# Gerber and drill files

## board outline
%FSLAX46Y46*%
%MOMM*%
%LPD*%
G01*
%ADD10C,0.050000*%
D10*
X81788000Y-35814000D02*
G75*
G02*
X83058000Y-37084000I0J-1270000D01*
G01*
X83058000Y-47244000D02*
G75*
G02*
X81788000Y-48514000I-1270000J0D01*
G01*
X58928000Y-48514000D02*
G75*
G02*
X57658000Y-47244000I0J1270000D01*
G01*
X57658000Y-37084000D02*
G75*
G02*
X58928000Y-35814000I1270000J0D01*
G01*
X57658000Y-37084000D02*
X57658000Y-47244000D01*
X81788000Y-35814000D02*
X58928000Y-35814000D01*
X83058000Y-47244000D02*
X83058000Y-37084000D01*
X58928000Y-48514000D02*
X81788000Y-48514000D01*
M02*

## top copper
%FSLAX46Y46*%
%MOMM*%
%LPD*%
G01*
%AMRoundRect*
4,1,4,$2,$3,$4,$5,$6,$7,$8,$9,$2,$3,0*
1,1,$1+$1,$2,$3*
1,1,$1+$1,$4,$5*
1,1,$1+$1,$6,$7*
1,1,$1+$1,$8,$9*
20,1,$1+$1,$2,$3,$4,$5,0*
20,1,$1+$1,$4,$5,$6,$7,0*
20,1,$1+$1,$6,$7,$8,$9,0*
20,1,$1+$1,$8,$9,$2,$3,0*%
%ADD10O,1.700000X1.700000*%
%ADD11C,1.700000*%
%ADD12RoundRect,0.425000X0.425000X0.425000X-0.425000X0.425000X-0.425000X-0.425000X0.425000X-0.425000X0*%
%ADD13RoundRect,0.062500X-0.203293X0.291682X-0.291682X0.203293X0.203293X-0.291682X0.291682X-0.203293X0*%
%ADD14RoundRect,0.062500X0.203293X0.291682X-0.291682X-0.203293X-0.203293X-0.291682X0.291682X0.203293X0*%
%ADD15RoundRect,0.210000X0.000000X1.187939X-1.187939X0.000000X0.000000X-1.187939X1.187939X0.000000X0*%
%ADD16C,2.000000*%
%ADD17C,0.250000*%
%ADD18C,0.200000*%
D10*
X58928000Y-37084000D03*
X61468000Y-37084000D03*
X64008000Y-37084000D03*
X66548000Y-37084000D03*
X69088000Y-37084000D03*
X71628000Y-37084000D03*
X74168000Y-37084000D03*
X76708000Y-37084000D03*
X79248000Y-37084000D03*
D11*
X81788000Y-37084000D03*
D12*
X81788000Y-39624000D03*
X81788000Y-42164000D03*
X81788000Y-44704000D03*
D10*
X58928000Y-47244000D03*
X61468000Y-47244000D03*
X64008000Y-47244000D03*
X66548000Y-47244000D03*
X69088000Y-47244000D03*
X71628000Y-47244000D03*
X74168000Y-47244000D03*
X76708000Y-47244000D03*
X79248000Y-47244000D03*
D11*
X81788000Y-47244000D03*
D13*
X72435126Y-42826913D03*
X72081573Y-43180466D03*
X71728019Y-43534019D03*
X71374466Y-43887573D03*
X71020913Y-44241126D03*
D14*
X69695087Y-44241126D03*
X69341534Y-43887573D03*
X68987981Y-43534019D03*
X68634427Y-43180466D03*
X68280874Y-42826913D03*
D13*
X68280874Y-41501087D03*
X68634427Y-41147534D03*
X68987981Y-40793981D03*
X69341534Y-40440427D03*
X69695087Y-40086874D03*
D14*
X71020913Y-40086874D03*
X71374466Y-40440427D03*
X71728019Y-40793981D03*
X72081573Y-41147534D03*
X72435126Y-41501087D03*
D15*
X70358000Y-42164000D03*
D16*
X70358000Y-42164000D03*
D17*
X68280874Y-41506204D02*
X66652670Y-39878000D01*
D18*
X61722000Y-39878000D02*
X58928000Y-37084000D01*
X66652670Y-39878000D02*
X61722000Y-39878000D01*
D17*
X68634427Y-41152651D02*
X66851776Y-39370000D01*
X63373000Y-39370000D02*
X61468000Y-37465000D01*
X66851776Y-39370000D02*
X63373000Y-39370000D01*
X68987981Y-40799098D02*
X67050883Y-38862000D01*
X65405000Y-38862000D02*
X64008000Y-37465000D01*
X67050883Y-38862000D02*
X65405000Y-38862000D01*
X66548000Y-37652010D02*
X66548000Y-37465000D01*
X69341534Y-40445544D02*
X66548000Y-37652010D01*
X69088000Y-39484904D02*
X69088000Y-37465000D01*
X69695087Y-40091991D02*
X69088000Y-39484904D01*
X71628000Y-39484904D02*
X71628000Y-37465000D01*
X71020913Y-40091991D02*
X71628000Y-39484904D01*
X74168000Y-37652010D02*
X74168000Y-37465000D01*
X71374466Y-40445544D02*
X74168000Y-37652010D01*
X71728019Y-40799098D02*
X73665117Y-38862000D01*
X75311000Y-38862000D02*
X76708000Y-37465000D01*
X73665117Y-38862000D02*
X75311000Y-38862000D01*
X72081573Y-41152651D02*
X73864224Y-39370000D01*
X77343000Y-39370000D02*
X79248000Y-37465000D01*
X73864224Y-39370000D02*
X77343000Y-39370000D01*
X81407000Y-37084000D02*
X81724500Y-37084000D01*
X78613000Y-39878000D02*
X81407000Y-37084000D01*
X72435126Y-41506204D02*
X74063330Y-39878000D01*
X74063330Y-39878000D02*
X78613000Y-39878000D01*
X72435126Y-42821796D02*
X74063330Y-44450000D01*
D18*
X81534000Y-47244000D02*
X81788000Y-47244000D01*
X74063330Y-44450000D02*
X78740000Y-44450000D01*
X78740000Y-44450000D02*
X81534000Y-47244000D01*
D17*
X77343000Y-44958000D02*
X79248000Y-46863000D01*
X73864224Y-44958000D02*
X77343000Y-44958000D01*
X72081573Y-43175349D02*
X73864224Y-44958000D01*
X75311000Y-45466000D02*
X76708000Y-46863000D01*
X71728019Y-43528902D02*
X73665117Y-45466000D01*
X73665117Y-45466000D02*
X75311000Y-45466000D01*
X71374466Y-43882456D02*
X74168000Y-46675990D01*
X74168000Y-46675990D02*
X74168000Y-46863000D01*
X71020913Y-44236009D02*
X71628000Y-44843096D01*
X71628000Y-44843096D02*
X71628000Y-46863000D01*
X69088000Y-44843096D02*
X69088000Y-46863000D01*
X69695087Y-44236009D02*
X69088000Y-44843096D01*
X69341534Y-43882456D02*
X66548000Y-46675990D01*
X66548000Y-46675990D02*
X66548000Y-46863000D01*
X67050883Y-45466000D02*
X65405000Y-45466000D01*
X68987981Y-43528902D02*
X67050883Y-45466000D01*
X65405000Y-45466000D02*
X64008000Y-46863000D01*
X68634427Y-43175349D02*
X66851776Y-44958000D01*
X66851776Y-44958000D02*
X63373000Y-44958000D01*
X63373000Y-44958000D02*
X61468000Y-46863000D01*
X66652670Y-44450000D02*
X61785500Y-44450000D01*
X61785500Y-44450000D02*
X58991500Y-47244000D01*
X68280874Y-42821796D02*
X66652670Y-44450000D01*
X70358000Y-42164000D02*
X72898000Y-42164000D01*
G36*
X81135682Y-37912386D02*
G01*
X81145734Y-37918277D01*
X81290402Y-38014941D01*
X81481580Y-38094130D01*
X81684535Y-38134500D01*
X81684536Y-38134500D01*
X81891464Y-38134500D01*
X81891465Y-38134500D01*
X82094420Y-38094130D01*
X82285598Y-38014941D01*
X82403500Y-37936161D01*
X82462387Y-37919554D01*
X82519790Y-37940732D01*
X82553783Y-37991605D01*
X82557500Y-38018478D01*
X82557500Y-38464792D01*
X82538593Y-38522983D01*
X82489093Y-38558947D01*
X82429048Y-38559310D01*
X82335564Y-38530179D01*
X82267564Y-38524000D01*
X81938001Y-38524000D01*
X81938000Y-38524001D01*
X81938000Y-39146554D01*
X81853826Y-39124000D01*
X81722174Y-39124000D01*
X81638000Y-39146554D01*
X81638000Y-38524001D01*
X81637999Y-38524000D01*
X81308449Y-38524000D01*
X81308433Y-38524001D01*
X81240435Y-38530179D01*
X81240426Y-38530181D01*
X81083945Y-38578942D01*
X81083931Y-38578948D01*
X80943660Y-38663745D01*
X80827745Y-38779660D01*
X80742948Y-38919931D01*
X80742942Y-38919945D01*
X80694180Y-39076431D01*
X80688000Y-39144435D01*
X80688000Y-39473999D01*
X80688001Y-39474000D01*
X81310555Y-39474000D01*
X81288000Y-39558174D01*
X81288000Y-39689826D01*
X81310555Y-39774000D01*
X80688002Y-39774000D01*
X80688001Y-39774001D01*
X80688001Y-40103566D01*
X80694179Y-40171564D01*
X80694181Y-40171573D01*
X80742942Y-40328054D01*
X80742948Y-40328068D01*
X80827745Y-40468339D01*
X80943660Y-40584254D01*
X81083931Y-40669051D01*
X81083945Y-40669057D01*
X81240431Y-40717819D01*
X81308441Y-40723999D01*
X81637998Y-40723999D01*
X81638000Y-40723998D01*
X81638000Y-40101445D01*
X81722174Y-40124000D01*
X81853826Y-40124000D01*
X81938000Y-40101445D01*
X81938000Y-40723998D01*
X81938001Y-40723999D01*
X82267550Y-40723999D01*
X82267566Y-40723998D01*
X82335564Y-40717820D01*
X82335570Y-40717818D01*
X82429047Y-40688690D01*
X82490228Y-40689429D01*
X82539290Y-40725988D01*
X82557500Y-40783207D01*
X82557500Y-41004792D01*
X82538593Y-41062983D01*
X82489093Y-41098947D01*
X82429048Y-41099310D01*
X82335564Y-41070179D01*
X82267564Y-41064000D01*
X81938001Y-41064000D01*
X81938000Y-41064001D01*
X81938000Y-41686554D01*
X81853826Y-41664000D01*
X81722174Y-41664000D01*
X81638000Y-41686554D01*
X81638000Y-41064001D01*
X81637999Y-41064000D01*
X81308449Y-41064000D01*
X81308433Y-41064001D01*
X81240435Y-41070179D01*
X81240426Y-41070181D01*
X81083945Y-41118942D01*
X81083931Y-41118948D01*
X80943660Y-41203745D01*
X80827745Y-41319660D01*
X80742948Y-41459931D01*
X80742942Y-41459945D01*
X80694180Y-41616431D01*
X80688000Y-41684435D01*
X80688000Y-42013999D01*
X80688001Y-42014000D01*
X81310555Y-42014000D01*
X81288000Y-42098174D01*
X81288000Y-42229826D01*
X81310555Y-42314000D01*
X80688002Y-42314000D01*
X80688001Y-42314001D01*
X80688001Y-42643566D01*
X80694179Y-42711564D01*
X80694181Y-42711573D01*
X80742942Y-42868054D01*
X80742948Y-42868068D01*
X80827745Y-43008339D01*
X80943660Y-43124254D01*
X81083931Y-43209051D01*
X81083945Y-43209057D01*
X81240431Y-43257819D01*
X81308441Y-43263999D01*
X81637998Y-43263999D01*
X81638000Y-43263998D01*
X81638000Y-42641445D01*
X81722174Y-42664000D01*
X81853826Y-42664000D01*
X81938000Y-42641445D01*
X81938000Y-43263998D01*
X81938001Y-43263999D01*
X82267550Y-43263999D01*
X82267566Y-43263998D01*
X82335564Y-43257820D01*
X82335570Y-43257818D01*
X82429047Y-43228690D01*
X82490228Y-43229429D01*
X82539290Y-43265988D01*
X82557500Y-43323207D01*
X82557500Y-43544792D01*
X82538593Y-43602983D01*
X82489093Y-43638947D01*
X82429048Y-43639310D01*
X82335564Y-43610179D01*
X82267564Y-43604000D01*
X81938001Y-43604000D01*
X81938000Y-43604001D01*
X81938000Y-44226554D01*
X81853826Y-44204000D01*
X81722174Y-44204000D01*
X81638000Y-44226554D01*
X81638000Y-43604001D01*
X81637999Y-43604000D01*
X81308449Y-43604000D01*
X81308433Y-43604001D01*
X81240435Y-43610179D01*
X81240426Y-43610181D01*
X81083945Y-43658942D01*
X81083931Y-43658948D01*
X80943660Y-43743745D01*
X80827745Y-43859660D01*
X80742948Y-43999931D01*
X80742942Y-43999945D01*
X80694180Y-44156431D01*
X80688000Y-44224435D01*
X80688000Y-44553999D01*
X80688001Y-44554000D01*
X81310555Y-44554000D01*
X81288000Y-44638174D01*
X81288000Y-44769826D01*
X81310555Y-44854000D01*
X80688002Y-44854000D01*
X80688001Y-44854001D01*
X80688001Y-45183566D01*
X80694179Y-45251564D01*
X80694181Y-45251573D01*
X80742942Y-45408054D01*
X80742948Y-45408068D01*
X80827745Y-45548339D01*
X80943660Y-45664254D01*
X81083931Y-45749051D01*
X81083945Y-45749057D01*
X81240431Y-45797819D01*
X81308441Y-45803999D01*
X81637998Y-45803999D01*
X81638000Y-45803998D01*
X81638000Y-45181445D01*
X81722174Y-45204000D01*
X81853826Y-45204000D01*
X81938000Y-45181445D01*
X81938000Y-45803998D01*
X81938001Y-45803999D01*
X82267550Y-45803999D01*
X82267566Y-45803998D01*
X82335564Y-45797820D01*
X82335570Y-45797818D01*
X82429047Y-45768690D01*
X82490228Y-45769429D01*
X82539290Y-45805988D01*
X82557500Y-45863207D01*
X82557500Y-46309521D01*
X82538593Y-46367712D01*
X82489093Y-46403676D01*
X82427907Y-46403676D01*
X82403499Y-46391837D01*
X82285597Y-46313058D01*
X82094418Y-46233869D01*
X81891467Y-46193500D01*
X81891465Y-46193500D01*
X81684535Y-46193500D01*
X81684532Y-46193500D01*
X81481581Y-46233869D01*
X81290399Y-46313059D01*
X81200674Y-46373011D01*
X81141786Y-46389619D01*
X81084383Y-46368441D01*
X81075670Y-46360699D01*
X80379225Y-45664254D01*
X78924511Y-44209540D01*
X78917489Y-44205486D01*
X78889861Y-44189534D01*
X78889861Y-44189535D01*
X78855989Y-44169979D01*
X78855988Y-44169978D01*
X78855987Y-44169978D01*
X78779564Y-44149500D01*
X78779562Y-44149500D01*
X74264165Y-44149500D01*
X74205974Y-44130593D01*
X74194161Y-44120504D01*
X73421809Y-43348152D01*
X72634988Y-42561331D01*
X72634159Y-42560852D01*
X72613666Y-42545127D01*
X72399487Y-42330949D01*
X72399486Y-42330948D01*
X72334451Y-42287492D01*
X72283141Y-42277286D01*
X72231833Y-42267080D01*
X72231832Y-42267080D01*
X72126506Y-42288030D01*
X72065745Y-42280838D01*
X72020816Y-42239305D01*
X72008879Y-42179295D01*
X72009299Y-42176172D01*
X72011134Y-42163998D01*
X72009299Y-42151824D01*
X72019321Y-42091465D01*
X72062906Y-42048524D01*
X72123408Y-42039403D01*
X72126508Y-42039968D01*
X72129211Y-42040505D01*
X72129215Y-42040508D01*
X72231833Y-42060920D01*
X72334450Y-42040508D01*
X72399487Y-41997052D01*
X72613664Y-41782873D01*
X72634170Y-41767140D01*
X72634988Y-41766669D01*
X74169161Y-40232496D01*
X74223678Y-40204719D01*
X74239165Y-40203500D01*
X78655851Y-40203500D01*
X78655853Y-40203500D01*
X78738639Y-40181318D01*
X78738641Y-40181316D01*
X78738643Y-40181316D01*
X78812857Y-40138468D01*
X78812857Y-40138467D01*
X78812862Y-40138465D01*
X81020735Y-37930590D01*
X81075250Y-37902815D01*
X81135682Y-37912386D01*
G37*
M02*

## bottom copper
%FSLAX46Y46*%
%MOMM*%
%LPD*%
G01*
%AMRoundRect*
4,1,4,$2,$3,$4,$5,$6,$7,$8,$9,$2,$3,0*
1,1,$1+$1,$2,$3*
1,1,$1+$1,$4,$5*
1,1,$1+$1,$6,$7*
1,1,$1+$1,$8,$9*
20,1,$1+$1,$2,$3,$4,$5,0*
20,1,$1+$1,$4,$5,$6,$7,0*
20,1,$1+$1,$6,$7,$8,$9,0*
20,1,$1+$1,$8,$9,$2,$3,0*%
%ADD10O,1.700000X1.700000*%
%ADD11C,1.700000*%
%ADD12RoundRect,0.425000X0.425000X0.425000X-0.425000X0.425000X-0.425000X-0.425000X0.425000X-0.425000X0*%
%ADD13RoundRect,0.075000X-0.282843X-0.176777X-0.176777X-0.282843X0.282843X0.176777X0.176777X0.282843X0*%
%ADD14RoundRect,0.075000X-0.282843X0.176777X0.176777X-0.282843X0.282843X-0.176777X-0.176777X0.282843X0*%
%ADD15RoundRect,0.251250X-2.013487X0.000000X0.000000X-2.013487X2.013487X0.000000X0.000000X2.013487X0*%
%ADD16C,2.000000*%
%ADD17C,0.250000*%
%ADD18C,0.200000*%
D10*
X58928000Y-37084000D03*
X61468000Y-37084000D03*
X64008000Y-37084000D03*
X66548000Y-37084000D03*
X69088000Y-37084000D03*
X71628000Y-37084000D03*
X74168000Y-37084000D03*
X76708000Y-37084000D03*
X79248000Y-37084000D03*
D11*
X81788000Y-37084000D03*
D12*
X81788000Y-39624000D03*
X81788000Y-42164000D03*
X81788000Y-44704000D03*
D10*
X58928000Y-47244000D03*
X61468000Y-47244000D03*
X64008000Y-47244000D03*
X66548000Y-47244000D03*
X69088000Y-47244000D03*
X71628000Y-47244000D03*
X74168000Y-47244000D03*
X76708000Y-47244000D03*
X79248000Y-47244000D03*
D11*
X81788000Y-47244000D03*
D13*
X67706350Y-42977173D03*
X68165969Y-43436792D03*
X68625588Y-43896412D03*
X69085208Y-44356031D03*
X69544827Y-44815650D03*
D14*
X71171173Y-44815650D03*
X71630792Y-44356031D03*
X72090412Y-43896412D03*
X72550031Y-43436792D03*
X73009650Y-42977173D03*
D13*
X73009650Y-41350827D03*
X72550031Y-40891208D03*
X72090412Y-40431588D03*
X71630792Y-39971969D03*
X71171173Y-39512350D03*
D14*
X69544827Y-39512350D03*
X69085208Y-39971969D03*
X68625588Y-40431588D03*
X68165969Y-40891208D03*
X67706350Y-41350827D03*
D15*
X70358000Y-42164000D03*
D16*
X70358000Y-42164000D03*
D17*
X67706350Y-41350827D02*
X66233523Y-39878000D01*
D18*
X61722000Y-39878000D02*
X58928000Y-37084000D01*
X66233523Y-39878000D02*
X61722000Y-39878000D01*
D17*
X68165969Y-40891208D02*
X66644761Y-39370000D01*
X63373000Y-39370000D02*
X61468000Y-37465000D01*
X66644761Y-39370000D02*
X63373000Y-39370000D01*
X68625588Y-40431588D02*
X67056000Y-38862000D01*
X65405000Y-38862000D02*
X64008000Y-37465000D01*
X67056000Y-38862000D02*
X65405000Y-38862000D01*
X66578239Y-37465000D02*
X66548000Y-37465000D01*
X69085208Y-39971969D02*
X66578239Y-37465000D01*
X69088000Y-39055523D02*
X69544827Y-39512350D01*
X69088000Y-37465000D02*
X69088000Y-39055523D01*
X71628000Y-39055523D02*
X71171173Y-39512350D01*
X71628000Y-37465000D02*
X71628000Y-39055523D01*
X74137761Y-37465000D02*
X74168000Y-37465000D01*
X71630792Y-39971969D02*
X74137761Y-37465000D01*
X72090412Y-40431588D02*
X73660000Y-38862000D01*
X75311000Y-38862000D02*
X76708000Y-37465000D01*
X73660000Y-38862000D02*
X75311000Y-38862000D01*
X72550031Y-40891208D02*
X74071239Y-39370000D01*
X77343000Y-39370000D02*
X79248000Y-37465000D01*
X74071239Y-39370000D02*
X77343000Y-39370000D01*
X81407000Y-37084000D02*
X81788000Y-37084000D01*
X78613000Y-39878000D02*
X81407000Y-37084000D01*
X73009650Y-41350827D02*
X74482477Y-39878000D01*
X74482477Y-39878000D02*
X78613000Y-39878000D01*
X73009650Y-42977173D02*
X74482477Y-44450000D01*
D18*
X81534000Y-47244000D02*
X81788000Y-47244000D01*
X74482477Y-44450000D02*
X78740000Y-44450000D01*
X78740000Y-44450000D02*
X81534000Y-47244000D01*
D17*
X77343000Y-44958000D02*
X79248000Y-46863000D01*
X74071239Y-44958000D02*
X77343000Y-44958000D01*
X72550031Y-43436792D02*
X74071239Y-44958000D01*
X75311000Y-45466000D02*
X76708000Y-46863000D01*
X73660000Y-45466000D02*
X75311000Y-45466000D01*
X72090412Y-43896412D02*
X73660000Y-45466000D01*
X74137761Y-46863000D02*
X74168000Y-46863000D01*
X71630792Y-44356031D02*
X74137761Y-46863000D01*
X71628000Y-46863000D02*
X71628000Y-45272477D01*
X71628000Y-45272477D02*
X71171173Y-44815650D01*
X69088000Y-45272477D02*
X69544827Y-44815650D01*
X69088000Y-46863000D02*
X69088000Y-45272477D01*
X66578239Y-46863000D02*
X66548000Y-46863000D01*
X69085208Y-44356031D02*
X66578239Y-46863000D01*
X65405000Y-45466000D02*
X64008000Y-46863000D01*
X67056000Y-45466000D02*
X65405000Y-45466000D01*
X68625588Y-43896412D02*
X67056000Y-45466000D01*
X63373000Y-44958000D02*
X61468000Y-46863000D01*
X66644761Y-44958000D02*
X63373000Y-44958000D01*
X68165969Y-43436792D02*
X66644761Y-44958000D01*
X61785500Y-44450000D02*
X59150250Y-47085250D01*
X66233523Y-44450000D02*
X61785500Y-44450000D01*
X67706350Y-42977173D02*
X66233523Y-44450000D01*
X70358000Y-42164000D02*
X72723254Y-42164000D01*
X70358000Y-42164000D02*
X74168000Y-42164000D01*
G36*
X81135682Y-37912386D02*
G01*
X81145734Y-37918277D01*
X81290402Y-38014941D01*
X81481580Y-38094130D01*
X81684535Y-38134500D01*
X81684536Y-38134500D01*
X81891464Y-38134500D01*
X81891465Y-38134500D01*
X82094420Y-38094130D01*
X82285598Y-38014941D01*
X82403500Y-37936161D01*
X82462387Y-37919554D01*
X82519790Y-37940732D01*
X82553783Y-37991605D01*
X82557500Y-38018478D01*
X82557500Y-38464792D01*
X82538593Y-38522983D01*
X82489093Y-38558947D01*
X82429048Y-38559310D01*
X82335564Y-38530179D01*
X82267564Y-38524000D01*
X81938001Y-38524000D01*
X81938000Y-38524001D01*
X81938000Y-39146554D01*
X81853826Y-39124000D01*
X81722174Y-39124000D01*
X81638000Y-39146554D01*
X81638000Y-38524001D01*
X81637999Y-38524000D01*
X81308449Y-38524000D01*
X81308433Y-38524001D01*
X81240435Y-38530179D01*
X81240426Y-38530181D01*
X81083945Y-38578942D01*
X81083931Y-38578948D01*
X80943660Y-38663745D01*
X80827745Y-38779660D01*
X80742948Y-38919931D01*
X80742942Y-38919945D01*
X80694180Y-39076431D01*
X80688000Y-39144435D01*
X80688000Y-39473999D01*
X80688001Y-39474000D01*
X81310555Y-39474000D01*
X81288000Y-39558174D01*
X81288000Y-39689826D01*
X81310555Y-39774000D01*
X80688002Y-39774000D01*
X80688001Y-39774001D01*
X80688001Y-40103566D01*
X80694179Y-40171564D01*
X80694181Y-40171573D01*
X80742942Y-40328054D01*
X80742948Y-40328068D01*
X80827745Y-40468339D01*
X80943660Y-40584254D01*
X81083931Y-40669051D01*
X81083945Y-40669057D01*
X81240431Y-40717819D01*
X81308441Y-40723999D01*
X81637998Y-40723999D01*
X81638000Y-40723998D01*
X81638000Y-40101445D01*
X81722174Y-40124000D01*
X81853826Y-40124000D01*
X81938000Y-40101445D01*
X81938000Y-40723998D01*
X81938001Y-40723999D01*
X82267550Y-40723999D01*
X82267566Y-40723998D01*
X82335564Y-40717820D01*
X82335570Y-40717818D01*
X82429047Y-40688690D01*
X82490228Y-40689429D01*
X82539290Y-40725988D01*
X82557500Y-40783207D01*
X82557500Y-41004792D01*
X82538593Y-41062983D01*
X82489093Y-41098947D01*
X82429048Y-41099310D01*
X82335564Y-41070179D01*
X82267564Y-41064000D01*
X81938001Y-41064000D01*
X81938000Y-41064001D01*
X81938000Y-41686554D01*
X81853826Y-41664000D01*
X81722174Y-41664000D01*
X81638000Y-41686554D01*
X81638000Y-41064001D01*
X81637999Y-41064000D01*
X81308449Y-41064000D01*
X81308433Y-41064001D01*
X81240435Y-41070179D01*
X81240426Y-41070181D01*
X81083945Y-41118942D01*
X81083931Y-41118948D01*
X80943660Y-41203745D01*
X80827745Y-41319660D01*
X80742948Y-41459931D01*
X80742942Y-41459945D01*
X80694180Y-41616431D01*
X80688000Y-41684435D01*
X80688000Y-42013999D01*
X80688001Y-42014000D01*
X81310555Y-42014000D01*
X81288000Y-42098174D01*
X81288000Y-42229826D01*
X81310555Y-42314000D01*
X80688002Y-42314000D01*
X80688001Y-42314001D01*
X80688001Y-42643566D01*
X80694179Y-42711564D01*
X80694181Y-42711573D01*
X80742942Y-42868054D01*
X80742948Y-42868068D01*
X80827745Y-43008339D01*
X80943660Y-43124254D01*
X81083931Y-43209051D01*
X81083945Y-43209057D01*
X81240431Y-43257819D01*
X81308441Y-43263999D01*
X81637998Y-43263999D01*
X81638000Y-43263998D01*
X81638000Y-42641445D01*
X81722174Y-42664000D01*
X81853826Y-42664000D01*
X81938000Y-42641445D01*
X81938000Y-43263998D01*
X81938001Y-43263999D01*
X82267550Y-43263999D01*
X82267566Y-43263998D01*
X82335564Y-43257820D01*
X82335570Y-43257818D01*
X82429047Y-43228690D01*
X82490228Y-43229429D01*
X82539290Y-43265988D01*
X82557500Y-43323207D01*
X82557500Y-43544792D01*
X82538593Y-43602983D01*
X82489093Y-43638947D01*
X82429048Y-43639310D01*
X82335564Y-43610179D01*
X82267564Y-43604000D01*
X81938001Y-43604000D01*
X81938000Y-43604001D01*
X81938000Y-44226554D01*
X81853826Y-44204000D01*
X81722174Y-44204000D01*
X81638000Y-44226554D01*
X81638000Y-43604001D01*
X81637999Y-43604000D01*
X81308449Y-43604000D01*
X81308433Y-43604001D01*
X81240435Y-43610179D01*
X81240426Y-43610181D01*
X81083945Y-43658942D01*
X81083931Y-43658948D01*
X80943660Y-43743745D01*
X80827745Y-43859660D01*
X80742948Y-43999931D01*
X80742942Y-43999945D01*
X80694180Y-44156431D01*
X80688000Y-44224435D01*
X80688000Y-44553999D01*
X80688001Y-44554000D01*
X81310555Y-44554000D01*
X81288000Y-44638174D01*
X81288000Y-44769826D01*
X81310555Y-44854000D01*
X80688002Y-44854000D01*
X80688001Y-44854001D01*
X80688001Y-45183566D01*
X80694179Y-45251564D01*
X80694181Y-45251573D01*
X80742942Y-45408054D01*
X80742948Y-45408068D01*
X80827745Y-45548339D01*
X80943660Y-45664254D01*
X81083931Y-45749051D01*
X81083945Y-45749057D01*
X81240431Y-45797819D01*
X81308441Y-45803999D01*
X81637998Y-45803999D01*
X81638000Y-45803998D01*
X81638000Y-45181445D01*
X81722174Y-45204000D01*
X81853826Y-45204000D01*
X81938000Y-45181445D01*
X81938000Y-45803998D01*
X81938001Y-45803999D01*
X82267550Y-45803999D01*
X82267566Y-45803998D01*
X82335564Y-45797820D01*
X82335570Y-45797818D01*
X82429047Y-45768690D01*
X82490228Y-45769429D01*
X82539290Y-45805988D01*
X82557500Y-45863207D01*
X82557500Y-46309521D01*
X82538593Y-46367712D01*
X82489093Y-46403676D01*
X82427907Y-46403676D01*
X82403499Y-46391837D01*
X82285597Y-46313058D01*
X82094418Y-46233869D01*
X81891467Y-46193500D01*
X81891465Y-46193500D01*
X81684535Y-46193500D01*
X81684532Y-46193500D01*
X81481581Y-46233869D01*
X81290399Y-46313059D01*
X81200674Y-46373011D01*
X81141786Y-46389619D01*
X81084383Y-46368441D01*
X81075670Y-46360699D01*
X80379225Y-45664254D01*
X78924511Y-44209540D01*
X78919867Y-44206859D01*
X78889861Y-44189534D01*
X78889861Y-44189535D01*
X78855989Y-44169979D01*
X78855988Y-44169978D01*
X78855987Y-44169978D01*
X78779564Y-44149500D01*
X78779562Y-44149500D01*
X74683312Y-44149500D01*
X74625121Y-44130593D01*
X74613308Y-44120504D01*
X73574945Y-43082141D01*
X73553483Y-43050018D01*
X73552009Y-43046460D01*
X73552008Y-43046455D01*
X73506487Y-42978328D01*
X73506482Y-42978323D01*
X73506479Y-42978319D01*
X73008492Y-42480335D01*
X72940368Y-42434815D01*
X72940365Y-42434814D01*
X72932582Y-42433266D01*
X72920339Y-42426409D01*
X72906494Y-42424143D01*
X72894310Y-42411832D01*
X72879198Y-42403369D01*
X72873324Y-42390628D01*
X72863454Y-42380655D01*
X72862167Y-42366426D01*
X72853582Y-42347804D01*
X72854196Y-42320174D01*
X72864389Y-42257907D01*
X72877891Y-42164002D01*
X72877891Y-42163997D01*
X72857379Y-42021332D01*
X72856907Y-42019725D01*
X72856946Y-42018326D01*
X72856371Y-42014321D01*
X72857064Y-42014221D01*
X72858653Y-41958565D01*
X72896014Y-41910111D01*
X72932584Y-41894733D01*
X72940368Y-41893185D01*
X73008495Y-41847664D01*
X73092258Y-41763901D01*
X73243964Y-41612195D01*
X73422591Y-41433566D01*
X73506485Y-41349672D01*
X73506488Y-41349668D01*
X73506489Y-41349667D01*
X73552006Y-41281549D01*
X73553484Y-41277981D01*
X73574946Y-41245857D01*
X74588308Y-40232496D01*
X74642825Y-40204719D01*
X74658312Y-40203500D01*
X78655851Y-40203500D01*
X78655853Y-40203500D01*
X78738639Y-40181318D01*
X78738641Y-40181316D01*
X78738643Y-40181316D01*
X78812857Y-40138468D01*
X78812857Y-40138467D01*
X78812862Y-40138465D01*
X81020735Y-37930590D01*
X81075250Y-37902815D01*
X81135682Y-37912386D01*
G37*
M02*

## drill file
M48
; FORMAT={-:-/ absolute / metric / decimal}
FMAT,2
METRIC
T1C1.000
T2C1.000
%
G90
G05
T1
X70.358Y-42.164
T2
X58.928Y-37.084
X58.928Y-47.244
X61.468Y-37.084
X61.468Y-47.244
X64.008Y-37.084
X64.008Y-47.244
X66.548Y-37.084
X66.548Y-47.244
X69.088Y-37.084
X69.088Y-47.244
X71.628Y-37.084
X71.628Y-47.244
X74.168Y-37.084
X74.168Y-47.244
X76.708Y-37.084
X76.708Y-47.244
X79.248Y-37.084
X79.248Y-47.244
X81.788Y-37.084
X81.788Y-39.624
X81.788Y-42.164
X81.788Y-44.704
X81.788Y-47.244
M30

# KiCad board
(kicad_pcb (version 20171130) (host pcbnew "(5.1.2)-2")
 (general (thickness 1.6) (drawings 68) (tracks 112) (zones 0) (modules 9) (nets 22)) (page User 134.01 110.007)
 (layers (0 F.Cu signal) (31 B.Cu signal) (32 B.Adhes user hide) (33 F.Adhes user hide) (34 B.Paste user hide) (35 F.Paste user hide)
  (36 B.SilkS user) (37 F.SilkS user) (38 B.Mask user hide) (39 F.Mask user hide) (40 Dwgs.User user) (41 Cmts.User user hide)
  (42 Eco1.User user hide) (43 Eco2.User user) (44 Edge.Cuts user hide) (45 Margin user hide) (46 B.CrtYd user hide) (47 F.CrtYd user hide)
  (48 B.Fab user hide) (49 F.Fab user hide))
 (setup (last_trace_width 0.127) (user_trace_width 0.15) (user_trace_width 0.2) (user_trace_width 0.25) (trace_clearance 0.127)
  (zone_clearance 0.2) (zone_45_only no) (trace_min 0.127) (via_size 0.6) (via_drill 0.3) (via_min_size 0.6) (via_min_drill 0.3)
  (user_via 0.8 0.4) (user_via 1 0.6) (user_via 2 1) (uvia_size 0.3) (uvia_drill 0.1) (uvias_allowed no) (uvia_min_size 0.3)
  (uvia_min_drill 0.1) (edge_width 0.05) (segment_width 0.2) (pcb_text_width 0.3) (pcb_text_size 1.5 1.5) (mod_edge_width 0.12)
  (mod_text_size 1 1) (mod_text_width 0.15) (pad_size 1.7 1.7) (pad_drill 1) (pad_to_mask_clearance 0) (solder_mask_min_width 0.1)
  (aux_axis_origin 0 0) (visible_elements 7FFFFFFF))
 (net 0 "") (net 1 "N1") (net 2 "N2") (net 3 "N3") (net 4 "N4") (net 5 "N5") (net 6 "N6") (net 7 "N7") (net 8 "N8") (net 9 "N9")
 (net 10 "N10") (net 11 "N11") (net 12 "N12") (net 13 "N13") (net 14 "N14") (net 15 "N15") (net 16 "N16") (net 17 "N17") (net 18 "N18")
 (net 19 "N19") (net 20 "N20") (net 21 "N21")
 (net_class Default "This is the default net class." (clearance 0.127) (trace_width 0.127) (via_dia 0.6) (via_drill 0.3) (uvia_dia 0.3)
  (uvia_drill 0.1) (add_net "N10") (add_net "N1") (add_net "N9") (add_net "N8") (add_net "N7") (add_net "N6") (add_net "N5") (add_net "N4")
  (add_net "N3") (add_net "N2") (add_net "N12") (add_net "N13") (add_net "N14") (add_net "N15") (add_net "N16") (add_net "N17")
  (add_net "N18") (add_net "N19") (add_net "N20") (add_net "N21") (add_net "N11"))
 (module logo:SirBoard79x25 (layer B.Cu) (at 62.738 43.688)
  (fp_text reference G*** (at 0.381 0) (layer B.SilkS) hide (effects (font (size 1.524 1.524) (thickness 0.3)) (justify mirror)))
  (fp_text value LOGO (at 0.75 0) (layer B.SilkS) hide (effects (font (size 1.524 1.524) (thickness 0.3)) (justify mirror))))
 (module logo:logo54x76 (layer B.Cu) (at 76.708 42.164)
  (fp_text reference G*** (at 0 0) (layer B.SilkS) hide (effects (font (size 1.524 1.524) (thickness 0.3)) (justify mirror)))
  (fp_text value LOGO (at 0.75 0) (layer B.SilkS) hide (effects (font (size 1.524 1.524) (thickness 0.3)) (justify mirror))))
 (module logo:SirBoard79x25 (layer F.Cu) (at 62.738 43.688)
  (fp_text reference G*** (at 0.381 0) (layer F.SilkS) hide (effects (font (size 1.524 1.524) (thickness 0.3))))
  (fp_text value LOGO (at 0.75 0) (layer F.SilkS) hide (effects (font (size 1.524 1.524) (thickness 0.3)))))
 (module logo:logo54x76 (layer F.Cu) (at 76.708 42.164)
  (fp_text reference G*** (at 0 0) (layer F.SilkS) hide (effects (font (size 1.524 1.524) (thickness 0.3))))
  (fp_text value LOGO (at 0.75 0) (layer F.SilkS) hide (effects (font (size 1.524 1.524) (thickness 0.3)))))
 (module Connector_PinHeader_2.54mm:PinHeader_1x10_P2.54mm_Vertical (layer F.Cu) (at 81.788 37.084 270)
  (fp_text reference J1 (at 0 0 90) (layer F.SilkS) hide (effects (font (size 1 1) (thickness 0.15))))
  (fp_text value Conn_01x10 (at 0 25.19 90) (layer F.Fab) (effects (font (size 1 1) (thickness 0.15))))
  (pad 10 thru_hole oval (at 0 22.86 270) (size 1.7 1.7) (drill 1) (layers *.Cu *.Mask) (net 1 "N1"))
  (pad 9 thru_hole oval (at 0 20.32 270) (size 1.7 1.7) (drill 1) (layers *.Cu *.Mask) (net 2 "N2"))
  (pad 8 thru_hole oval (at 0 17.78 270) (size 1.7 1.7) (drill 1) (layers *.Cu *.Mask) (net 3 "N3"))
  (pad 7 thru_hole oval (at 0 15.24 270) (size 1.7 1.7) (drill 1) (layers *.Cu *.Mask) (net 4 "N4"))
  (pad 6 thru_hole oval (at 0 12.7 270) (size 1.7 1.7) (drill 1) (layers *.Cu *.Mask) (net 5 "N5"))
  (pad 5 thru_hole oval (at 0 10.16 270) (size 1.7 1.7) (drill 1) (layers *.Cu *.Mask) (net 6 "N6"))
  (pad 4 thru_hole oval (at 0 7.62 270) (size 1.7 1.7) (drill 1) (layers *.Cu *.Mask) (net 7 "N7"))
  (pad 3 thru_hole oval (at 0 5.08 270) (size 1.7 1.7) (drill 1) (layers *.Cu *.Mask) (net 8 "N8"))
  (pad 2 thru_hole oval (at 0 2.54 270) (size 1.7 1.7) (drill 1) (layers *.Cu *.Mask) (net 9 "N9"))
  (pad 1 thru_hole circle (at 0 0 270) (size 1.7 1.7) (drill 1) (layers *.Cu *.Mask) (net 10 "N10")))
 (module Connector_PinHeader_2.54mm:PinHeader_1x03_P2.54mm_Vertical (layer B.Cu) (at 81.788 39.624 180)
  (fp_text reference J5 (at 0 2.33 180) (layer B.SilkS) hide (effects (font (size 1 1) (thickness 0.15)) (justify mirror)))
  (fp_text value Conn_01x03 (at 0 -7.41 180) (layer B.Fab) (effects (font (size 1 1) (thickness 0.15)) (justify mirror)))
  (pad 1 thru_hole roundrect (at 0 0 180) (size 1.7 1.7) (drill 1) (layers *.Cu *.Mask) (roundrect_rratio 0.25) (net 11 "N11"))
  (pad 2 thru_hole roundrect (at 0 -2.54 180) (size 1.7 1.7) (drill 1) (layers *.Cu *.Mask) (roundrect_rratio 0.25) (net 11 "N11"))
  (pad 3 thru_hole roundrect (at 0 -5.08 180) (size 1.7 1.7) (drill 1) (layers *.Cu *.Mask) (roundrect_rratio 0.25) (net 11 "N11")))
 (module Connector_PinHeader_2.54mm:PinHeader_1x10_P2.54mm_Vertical (layer F.Cu) (at 81.788 47.244 270)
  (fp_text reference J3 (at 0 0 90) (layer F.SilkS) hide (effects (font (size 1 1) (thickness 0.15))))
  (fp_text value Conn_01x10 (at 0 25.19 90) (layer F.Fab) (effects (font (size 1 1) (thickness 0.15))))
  (pad 10 thru_hole oval (at 0 22.86 270) (size 1.7 1.7) (drill 1) (layers *.Cu *.Mask) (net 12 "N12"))
  (pad 9 thru_hole oval (at 0 20.32 270) (size 1.7 1.7) (drill 1) (layers *.Cu *.Mask) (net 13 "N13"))
  (pad 8 thru_hole oval (at 0 17.78 270) (size 1.7 1.7) (drill 1) (layers *.Cu *.Mask) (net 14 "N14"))
  (pad 7 thru_hole oval (at 0 15.24 270) (size 1.7 1.7) (drill 1) (layers *.Cu *.Mask) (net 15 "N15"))
  (pad 6 thru_hole oval (at 0 12.7 270) (size 1.7 1.7) (drill 1) (layers *.Cu *.Mask) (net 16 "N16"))
  (pad 5 thru_hole oval (at 0 10.16 270) (size 1.7 1.7) (drill 1) (layers *.Cu *.Mask) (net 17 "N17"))
  (pad 4 thru_hole oval (at 0 7.62 270) (size 1.7 1.7) (drill 1) (layers *.Cu *.Mask) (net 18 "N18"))
  (pad 3 thru_hole oval (at 0 5.08 270) (size 1.7 1.7) (drill 1) (layers *.Cu *.Mask) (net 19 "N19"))
  (pad 2 thru_hole oval (at 0 2.54 270) (size 1.7 1.7) (drill 1) (layers *.Cu *.Mask) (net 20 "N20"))
  (pad 1 thru_hole circle (at 0 0 270) (size 1.7 1.7) (drill 1) (layers *.Cu *.Mask) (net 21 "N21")))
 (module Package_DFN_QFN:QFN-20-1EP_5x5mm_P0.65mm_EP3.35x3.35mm (layer B.Cu) (at 70.358 42.164 315)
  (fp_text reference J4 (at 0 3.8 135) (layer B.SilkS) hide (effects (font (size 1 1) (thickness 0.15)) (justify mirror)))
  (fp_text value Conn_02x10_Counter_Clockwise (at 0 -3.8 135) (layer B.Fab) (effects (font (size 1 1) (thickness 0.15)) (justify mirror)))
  (pad 20 smd roundrect (at -1.3 2.45 315) (size 0.3 0.8) (layers B.Cu B.Paste B.Mask) (roundrect_rratio 0.25) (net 12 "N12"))
  (pad 19 smd roundrect (at -0.65 2.45 315) (size 0.3 0.8) (layers B.Cu B.Paste B.Mask) (roundrect_rratio 0.25) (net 13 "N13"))
  (pad 18 smd roundrect (at 0 2.45 315) (size 0.3 0.8) (layers B.Cu B.Paste B.Mask) (roundrect_rratio 0.25) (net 14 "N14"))
  (pad 17 smd roundrect (at 0.65 2.45 315) (size 0.3 0.8) (layers B.Cu B.Paste B.Mask) (roundrect_rratio 0.25) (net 15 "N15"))
  (pad 16 smd roundrect (at 1.3 2.45 315) (size 0.3 0.8) (layers B.Cu B.Paste B.Mask) (roundrect_rratio 0.25) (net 16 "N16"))
  (pad 15 smd roundrect (at 2.45 1.3 315) (size 0.8 0.3) (layers B.Cu B.Paste B.Mask) (roundrect_rratio 0.25) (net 17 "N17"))
  (pad 14 smd roundrect (at 2.45 0.65 315) (size 0.8 0.3) (layers B.Cu B.Paste B.Mask) (roundrect_rratio 0.25) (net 18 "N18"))
  (pad 13 smd roundrect (at 2.45 0 315) (size 0.8 0.3) (layers B.Cu B.Paste B.Mask) (roundrect_rratio 0.25) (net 19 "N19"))
  (pad 12 smd roundrect (at 2.45 -0.65 315) (size 0.8 0.3) (layers B.Cu B.Paste B.Mask) (roundrect_rratio 0.25) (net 20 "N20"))
  (pad 11 smd roundrect (at 2.45 -1.3 315) (size 0.8 0.3) (layers B.Cu B.Paste B.Mask) (roundrect_rratio 0.25) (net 21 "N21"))
  (pad 10 smd roundrect (at 1.3 -2.45 315) (size 0.3 0.8) (layers B.Cu B.Paste B.Mask) (roundrect_rratio 0.25) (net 10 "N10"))
  (pad 9 smd roundrect (at 0.65 -2.45 315) (size 0.3 0.8) (layers B.Cu B.Paste B.Mask) (roundrect_rratio 0.25) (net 9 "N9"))
  (pad 8 smd roundrect (at 0 -2.45 315) (size 0.3 0.8) (layers B.Cu B.Paste B.Mask) (roundrect_rratio 0.25) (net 8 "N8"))
  (pad 7 smd roundrect (at -0.65 -2.45 315) (size 0.3 0.8) (layers B.Cu B.Paste B.Mask) (roundrect_rratio 0.25) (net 7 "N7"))
  (pad 6 smd roundrect (at -1.3 -2.45 315) (size 0.3 0.8) (layers B.Cu B.Paste B.Mask) (roundrect_rratio 0.25) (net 6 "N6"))
  (pad 5 smd roundrect (at -2.45 -1.3 315) (size 0.8 0.3) (layers B.Cu B.Paste B.Mask) (roundrect_rratio 0.25) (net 5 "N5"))
  (pad 4 smd roundrect (at -2.45 -0.65 315) (size 0.8 0.3) (layers B.Cu B.Paste B.Mask) (roundrect_rratio 0.25) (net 4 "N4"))
  (pad 3 smd roundrect (at -2.45 0 315) (size 0.8 0.3) (layers B.Cu B.Paste B.Mask) (roundrect_rratio 0.25) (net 3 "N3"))
  (pad 2 smd roundrect (at -2.45 0.65 315) (size 0.8 0.3) (layers B.Cu B.Paste B.Mask) (roundrect_rratio 0.25) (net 2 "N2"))
  (pad 1 smd roundrect (at -2.45 1.3 315) (size 0.8 0.3) (layers B.Cu B.Paste B.Mask) (roundrect_rratio 0.25) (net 1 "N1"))
  (pad "" smd roundrect (at 0.84 -0.84 315) (size 1.35 1.35) (layers B.Paste) (roundrect_rratio 0.185185))
  (pad "" smd roundrect (at 0.84 0.84 315) (size 1.35 1.35) (layers B.Paste) (roundrect_rratio 0.185185))
  (pad "" smd roundrect (at -0.84 -0.84 315) (size 1.35 1.35) (layers B.Paste) (roundrect_rratio 0.185185))
  (pad "" smd roundrect (at -0.84 0.84 315) (size 1.35 1.35) (layers B.Paste) (roundrect_rratio 0.185185))
  (pad 21 smd roundrect (at 0 0 315) (size 3.35 3.35) (layers B.Cu B.Mask) (roundrect_rratio 0.075) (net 11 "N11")))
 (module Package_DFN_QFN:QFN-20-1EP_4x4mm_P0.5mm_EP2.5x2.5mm (layer F.Cu) (at 70.358 42.164 225)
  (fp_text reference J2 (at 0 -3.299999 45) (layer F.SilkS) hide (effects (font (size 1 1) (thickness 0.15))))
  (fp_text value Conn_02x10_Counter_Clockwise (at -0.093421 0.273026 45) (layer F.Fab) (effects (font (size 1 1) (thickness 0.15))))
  (pad 20 smd roundrect (at -1 -1.9375 225) (size 0.25 0.825) (layers F.Cu F.Paste F.Mask) (roundrect_rratio 0.25) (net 21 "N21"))
  (pad 19 smd roundrect (at -0.5 -1.9375 225) (size 0.25 0.825) (layers F.Cu F.Paste F.Mask) (roundrect_rratio 0.25) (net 20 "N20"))
  (pad 18 smd roundrect (at 0 -1.9375 225) (size 0.25 0.825) (layers F.Cu F.Paste F.Mask) (roundrect_rratio 0.25) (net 19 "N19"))
  (pad 17 smd roundrect (at 0.5 -1.9375 225) (size 0.25 0.825) (layers F.Cu F.Paste F.Mask) (roundrect_rratio 0.25) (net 18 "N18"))
  (pad 16 smd roundrect (at 1 -1.9375 225) (size 0.25 0.825) (layers F.Cu F.Paste F.Mask) (roundrect_rratio 0.25) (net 17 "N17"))
  (pad 15 smd roundrect (at 1.9375 -1 225) (size 0.825 0.25) (layers F.Cu F.Paste F.Mask) (roundrect_rratio 0.25) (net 16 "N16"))
  (pad 14 smd roundrect (at 1.9375 -0.5 225) (size 0.825 0.25) (layers F.Cu F.Paste F.Mask) (roundrect_rratio 0.25) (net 15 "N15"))
  (pad 13 smd roundrect (at 1.9375 0 225) (size 0.825 0.25) (layers F.Cu F.Paste F.Mask) (roundrect_rratio 0.25) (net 14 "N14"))
  (pad 12 smd roundrect (at 1.9375 0.5 225) (size 0.825 0.25) (layers F.Cu F.Paste F.Mask) (roundrect_rratio 0.25) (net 13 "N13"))
  (pad 11 smd roundrect (at 1.9375 1 225) (size 0.825 0.25) (layers F.Cu F.Paste F.Mask) (roundrect_rratio 0.25) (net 12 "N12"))
  (pad 10 smd roundrect (at 1 1.9375 225) (size 0.25 0.825) (layers F.Cu F.Paste F.Mask) (roundrect_rratio 0.25) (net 1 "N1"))
  (pad 9 smd roundrect (at 0.5 1.9375 225) (size 0.25 0.825) (layers F.Cu F.Paste F.Mask) (roundrect_rratio 0.25) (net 2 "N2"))
  (pad 8 smd roundrect (at 0 1.9375 225) (size 0.25 0.825) (layers F.Cu F.Paste F.Mask) (roundrect_rratio 0.25) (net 3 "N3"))
  (pad 7 smd roundrect (at -0.5 1.9375 225) (size 0.25 0.825) (layers F.Cu F.Paste F.Mask) (roundrect_rratio 0.25) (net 4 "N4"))
  (pad 6 smd roundrect (at -1 1.9375 225) (size 0.25 0.825) (layers F.Cu F.Paste F.Mask) (roundrect_rratio 0.25) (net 5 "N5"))
  (pad 5 smd roundrect (at -1.9375 1 225) (size 0.825 0.25) (layers F.Cu F.Paste F.Mask) (roundrect_rratio 0.25) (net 6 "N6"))
  (pad 4 smd roundrect (at -1.9375 0.5 225) (size 0.825 0.25) (layers F.Cu F.Paste F.Mask) (roundrect_rratio 0.25) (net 7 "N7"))
  (pad 3 smd roundrect (at -1.9375 0 225) (size 0.825 0.25) (layers F.Cu F.Paste F.Mask) (roundrect_rratio 0.25) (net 8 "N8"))
  (pad 2 smd roundrect (at -1.9375 -0.5 225) (size 0.825 0.25) (layers F.Cu F.Paste F.Mask) (roundrect_rratio 0.25) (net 9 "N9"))
  (pad 1 smd roundrect (at -1.9375 -1 225) (size 0.825 0.25) (layers F.Cu F.Paste F.Mask) (roundrect_rratio 0.25) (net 10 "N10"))
  (pad "" smd roundrect (at 0.625 0.625 225) (size 1.01 1.01) (layers F.Paste) (roundrect_rratio 0.247525))
  (pad "" smd roundrect (at 0.625 -0.625 225) (size 1.01 1.01) (layers F.Paste) (roundrect_rratio 0.247525))
  (pad "" smd roundrect (at -0.625 0.625 225) (size 1.01 1.01) (layers F.Paste) (roundrect_rratio 0.247525))
  (pad "" smd roundrect (at -0.625 -0.625 225) (size 1.01 1.01) (layers F.Paste) (roundrect_rratio 0.247525))
  (pad 21 smd roundrect (at 0 0 225) (size 2.1 2.1) (layers F.Cu F.Mask) (roundrect_rratio 0.1) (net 11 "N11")))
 (gr_arc (start 81.788 37.084) (end 83.058 37.084) (angle -90) (layer Edge.Cuts) (width 0.05))
 (gr_arc (start 81.788 47.244) (end 81.788 48.514) (angle -90) (layer Edge.Cuts) (width 0.05))
 (gr_arc (start 58.928 47.244) (end 57.658 47.244) (angle -90) (layer Edge.Cuts) (width 0.05))
 (gr_arc (start 58.928 37.084) (end 58.928 35.814) (angle -90) (layer Edge.Cuts) (width 0.05))
 (gr_line (start 57.658 37.084) (end 57.658 47.244) (layer Edge.Cuts) (width 0.05))
 (gr_line (start 81.788 35.814) (end 58.928 35.814) (layer Edge.Cuts) (width 0.05))
 (gr_line (start 83.058 47.244) (end 83.058 37.084) (layer Edge.Cuts) (width 0.05))
 (gr_line (start 58.928 48.514) (end 81.788 48.514) (layer Edge.Cuts) (width 0.05))
 (segment (start 68.280874 41.506204) (end 66.65267 39.878) (width 0.25) (layer F.Cu) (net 1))
 (segment (start 67.70635 41.350827) (end 66.233523 39.878) (width 0.25) (layer B.Cu) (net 1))
 (segment (start 61.722 39.878) (end 58.928 37.084) (width 0.2) (layer B.Cu) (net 1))
 (segment (start 61.722 39.878) (end 58.928 37.084) (width 0.2) (layer F.Cu) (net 1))
 (segment (start 66.65267 39.878) (end 61.722 39.878) (width 0.2) (layer F.Cu) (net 1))
 (segment (start 66.233523 39.878) (end 61.722 39.878) (width 0.2) (layer B.Cu) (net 1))
 (segment (start 68.634427 41.152651) (end 66.851776 39.37) (width 0.25) (layer F.Cu) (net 2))
 (segment (start 63.373 39.37) (end 61.468 37.465) (width 0.25) (layer F.Cu) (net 2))
 (segment (start 66.851776 39.37) (end 63.373 39.37) (width 0.25) (layer F.Cu) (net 2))
 (segment (start 68.165969 40.891208) (end 66.644761 39.37) (width 0.25) (layer B.Cu) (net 2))
 (segment (start 63.373 39.37) (end 61.468 37.465) (width 0.25) (layer B.Cu) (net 2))
 (segment (start 66.644761 39.37) (end 63.373 39.37) (width 0.25) (layer B.Cu) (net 2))
 (segment (start 68.987981 40.799098) (end 67.050883 38.862) (width 0.25) (layer F.Cu) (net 3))
 (segment (start 65.405 38.862) (end 64.008 37.465) (width 0.25) (layer F.Cu) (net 3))
 (segment (start 67.050883 38.862) (end 65.405 38.862) (width 0.25) (layer F.Cu) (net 3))
 (segment (start 68.625588 40.431588) (end 67.056 38.862) (width 0.25) (layer B.Cu) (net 3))
 (segment (start 65.405 38.862) (end 64.008 37.465) (width 0.25) (layer B.Cu) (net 3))
 (segment (start 67.056 38.862) (end 65.405 38.862) (width 0.25) (layer B.Cu) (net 3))
 (segment (start 66.548 37.65201) (end 66.548 37.465) (width 0.25) (layer F.Cu) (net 4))
 (segment (start 69.341534 40.445544) (end 66.548 37.65201) (width 0.25) (layer F.Cu) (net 4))
 (segment (start 66.578239 37.465) (end 66.548 37.465) (width 0.25) (layer B.Cu) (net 4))
 (segment (start 69.085208 39.971969) (end 66.578239 37.465) (width 0.25) (layer B.Cu) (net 4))
 (segment (start 69.088 39.484904) (end 69.088 37.465) (width 0.25) (layer F.Cu) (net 5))
 (segment (start 69.695087 40.091991) (end 69.088 39.484904) (width 0.25) (layer F.Cu) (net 5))
 (segment (start 69.088 39.055523) (end 69.544827 39.51235) (width 0.25) (layer B.Cu) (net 5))
 (segment (start 69.088 37.465) (end 69.088 39.055523) (width 0.25) (layer B.Cu) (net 5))
 (segment (start 71.628 39.484904) (end 71.628 37.465) (width 0.25) (layer F.Cu) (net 6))
 (segment (start 71.020913 40.091991) (end 71.628 39.484904) (width 0.25) (layer F.Cu) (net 6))
 (segment (start 71.628 39.055523) (end 71.171173 39.51235) (width 0.25) (layer B.Cu) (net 6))
 (segment (start 71.628 37.465) (end 71.628 39.055523) (width 0.25) (layer B.Cu) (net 6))
 (segment (start 74.168 37.65201) (end 74.168 37.465) (width 0.25) (layer F.Cu) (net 7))
 (segment (start 71.374466 40.445544) (end 74.168 37.65201) (width 0.25) (layer F.Cu) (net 7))
 (segment (start 74.137761 37.465) (end 74.168 37.465) (width 0.25) (layer B.Cu) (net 7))
 (segment (start 71.630792 39.971969) (end 74.137761 37.465) (width 0.25) (layer B.Cu) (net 7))
 (segment (start 71.728019 40.799098) (end 73.665117 38.862) (width 0.25) (layer F.Cu) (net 8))
 (segment (start 75.311 38.862) (end 76.708 37.465) (width 0.25) (layer F.Cu) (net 8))
 (segment (start 73.665117 38.862) (end 75.311 38.862) (width 0.25) (layer F.Cu) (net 8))
 (segment (start 72.090412 40.431588) (end 73.66 38.862) (width 0.25) (layer B.Cu) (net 8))
 (segment (start 75.311 38.862) (end 76.708 37.465) (width 0.25) (layer B.Cu) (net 8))
 (segment (start 73.66 38.862) (end 75.311 38.862) (width 0.25) (layer B.Cu) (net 8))
 (segment (start 72.081573 41.152651) (end 73.864224 39.37) (width 0.25) (layer F.Cu) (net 9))
 (segment (start 77.343 39.37) (end 79.248 37.465) (width 0.25) (layer F.Cu) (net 9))
 (segment (start 73.864224 39.37) (end 77.343 39.37) (width 0.25) (layer F.Cu) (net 9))
 (segment (start 72.550031 40.891208) (end 74.071239 39.37) (width 0.25) (layer B.Cu) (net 9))
 (segment (start 77.343 39.37) (end 79.248 37.465) (width 0.25) (layer B.Cu) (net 9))
 (segment (start 74.071239 39.37) (end 77.343 39.37) (width 0.25) (layer B.Cu) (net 9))
 (segment (start 81.407 37.084) (end 81.788 37.084) (width 0.25) (layer B.Cu) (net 10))
 (segment (start 78.613 39.878) (end 81.407 37.084) (width 0.25) (layer B.Cu) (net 10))
 (segment (start 73.00965 41.350827) (end 74.482477 39.878) (width 0.25) (layer B.Cu) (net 10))
 (segment (start 74.482477 39.878) (end 78.613 39.878) (width 0.25) (layer B.Cu) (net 10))
 (segment (start 81.407 37.084) (end 81.7245 37.084) (width 0.25) (layer F.Cu) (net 10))
 (segment (start 78.613 39.878) (end 81.407 37.084) (width 0.25) (layer F.Cu) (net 10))
 (segment (start 72.435126 41.506204) (end 74.06333 39.878) (width 0.25) (layer F.Cu) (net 10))
 (segment (start 74.06333 39.878) (end 78.613 39.878) (width 0.25) (layer F.Cu) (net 10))
 (segment (start 73.00965 42.977173) (end 74.482477 44.45) (width 0.25) (layer B.Cu) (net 21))
 (segment (start 72.435126 42.821796) (end 74.06333 44.45) (width 0.25) (layer F.Cu) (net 21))
 (segment (start 81.534 47.244) (end 81.788 47.244) (width 0.2) (layer F.Cu) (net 21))
 (segment (start 74.06333 44.45) (end 78.74 44.45) (width 0.2) (layer F.Cu) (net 21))
 (segment (start 78.74 44.45) (end 81.534 47.244) (width 0.2) (layer F.Cu) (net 21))
 (segment (start 81.534 47.244) (end 81.788 47.244) (width 0.2) (layer B.Cu) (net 21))
 (segment (start 74.482477 44.45) (end 78.74 44.45) (width 0.2) (layer B.Cu) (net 21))
 (segment (start 78.74 44.45) (end 81.534 47.244) (width 0.2) (layer B.Cu) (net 21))
 (segment (start 77.343 44.958) (end 79.248 46.863) (width 0.25) (layer B.Cu) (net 20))
 (segment (start 74.071239 44.958) (end 77.343 44.958) (width 0.25) (layer B.Cu) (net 20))
 (segment (start 72.550031 43.436792) (end 74.071239 44.958) (width 0.25) (layer B.Cu) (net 20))
 (segment (start 77.343 44.958) (end 79.248 46.863) (width 0.25) (layer F.Cu) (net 20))
 (segment (start 73.864224 44.958) (end 77.343 44.958) (width 0.25) (layer F.Cu) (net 20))
 (segment (start 72.081573 43.175349) (end 73.864224 44.958) (width 0.25) (layer F.Cu) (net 20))
 (segment (start 75.311 45.466) (end 76.708 46.863) (width 0.25) (layer B.Cu) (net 19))
 (segment (start 73.66 45.466) (end 75.311 45.466) (width 0.25) (layer B.Cu) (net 19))
 (segment (start 72.090412 43.896412) (end 73.66 45.466) (width 0.25) (layer B.Cu) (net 19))
 (segment (start 75.311 45.466) (end 76.708 46.863) (width 0.25) (layer F.Cu) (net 19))
 (segment (start 71.728019 43.528902) (end 73.665117 45.466) (width 0.25) (layer F.Cu) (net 19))
 (segment (start 73.665117 45.466) (end 75.311 45.466) (width 0.25) (layer F.Cu) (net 19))
 (segment (start 74.137761 46.863) (end 74.168 46.863) (width 0.25) (layer B.Cu) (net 18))
 (segment (start 71.630792 44.356031) (end 74.137761 46.863) (width 0.25) (layer B.Cu) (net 18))
 (segment (start 71.374466 43.882456) (end 74.168 46.67599) (width 0.25) (layer F.Cu) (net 18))
 (segment (start 74.168 46.67599) (end 74.168 46.863) (width 0.25) (layer F.Cu) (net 18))
 (segment (start 71.628 46.863) (end 71.628 45.272477) (width 0.25) (layer B.Cu) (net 17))
 (segment (start 71.628 45.272477) (end 71.171173 44.81565) (width 0.25) (layer B.Cu) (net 17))
 (segment (start 71.020913 44.236009) (end 71.628 44.843096) (width 0.25) (layer F.Cu) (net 17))
 (segment (start 71.628 44.843096) (end 71.628 46.863) (width 0.25) (layer F.Cu) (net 17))
 (segment (start 69.088 45.272477) (end 69.544827 44.81565) (width 0.25) (layer B.Cu) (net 16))
 (segment (start 69.088 46.863) (end 69.088 45.272477) (width 0.25) (layer B.Cu) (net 16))
 (segment (start 69.088 44.843096) (end 69.088 46.863) (width 0.25) (layer F.Cu) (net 16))
 (segment (start 69.695087 44.236009) (end 69.088 44.843096) (width 0.25) (layer F.Cu) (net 16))
 (segment (start 66.578239 46.863) (end 66.548 46.863) (width 0.25) (layer B.Cu) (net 15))
 (segment (start 69.085208 44.356031) (end 66.578239 46.863) (width 0.25) (layer B.Cu) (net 15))
 (segment (start 69.341534 43.882456) (end 66.548 46.67599) (width 0.25) (layer F.Cu) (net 15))
 (segment (start 66.548 46.67599) (end 66.548 46.863) (width 0.25) (layer F.Cu) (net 15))
 (segment (start 65.405 45.466) (end 64.008 46.863) (width 0.25) (layer B.Cu) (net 14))
 (segment (start 67.056 45.466) (end 65.405 45.466) (width 0.25) (layer B.Cu) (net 14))
 (segment (start 68.625588 43.896412) (end 67.056 45.466) (width 0.25) (layer B.Cu) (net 14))
 (segment (start 67.050883 45.466) (end 65.405 45.466) (width 0.25) (layer F.Cu) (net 14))
 (segment (start 68.987981 43.528902) (end 67.050883 45.466) (width 0.25) (layer F.Cu) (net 14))
 (segment (start 65.405 45.466) (end 64.008 46.863) (width 0.25) (layer F.Cu) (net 14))
 (segment (start 63.373 44.958) (end 61.468 46.863) (width 0.25) (layer B.Cu) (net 13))
 (segment (start 66.644761 44.958) (end 63.373 44.958) (width 0.25) (layer B.Cu) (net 13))
 (segment (start 68.165969 43.436792) (end 66.644761 44.958) (width 0.25) (layer B.Cu) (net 13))
 (segment (start 68.634427 43.175349) (end 66.851776 44.958) (width 0.25) (layer F.Cu) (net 13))
 (segment (start 66.851776 44.958) (end 63.373 44.958) (width 0.25) (layer F.Cu) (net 13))
 (segment (start 63.373 44.958) (end 61.468 46.863) (width 0.25) (layer F.Cu) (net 13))
 (segment (start 66.65267 44.45) (end 61.7855 44.45) (width 0.25) (layer F.Cu) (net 12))
 (segment (start 61.7855 44.45) (end 58.9915 47.244) (width 0.25) (layer F.Cu) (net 12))
 (segment (start 61.7855 44.45) (end 59.15025 47.08525) (width 0.25) (layer B.Cu) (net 12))
 (segment (start 66.233523 44.45) (end 61.7855 44.45) (width 0.25) (layer B.Cu) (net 12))
 (segment (start 67.70635 42.977173) (end 66.233523 44.45) (width 0.25) (layer B.Cu) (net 12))
 (segment (start 68.280874 42.821796) (end 66.65267 44.45) (width 0.25) (layer F.Cu) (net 12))
 (via (at 70.358 42.164) (size 2) (drill 1) (layers F.Cu B.Cu) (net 11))
 (segment (start 70.358 42.164) (end 72.723254 42.164) (width 0.25) (layer B.Cu) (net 11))
 (segment (start 70.358 42.164) (end 74.168 42.164) (width 0.25) (layer B.Cu) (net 11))
 (segment (start 70.358 42.164) (end 72.898 42.164) (width 0.25) (layer F.Cu) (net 11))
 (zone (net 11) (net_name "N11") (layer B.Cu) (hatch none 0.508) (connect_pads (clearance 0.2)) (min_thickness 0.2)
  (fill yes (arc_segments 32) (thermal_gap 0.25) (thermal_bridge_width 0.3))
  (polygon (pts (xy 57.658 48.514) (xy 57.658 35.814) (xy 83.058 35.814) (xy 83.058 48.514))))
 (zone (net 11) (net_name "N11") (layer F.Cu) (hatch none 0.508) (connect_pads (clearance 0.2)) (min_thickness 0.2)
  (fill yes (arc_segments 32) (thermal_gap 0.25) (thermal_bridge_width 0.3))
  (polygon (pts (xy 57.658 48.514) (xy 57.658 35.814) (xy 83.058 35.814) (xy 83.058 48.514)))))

